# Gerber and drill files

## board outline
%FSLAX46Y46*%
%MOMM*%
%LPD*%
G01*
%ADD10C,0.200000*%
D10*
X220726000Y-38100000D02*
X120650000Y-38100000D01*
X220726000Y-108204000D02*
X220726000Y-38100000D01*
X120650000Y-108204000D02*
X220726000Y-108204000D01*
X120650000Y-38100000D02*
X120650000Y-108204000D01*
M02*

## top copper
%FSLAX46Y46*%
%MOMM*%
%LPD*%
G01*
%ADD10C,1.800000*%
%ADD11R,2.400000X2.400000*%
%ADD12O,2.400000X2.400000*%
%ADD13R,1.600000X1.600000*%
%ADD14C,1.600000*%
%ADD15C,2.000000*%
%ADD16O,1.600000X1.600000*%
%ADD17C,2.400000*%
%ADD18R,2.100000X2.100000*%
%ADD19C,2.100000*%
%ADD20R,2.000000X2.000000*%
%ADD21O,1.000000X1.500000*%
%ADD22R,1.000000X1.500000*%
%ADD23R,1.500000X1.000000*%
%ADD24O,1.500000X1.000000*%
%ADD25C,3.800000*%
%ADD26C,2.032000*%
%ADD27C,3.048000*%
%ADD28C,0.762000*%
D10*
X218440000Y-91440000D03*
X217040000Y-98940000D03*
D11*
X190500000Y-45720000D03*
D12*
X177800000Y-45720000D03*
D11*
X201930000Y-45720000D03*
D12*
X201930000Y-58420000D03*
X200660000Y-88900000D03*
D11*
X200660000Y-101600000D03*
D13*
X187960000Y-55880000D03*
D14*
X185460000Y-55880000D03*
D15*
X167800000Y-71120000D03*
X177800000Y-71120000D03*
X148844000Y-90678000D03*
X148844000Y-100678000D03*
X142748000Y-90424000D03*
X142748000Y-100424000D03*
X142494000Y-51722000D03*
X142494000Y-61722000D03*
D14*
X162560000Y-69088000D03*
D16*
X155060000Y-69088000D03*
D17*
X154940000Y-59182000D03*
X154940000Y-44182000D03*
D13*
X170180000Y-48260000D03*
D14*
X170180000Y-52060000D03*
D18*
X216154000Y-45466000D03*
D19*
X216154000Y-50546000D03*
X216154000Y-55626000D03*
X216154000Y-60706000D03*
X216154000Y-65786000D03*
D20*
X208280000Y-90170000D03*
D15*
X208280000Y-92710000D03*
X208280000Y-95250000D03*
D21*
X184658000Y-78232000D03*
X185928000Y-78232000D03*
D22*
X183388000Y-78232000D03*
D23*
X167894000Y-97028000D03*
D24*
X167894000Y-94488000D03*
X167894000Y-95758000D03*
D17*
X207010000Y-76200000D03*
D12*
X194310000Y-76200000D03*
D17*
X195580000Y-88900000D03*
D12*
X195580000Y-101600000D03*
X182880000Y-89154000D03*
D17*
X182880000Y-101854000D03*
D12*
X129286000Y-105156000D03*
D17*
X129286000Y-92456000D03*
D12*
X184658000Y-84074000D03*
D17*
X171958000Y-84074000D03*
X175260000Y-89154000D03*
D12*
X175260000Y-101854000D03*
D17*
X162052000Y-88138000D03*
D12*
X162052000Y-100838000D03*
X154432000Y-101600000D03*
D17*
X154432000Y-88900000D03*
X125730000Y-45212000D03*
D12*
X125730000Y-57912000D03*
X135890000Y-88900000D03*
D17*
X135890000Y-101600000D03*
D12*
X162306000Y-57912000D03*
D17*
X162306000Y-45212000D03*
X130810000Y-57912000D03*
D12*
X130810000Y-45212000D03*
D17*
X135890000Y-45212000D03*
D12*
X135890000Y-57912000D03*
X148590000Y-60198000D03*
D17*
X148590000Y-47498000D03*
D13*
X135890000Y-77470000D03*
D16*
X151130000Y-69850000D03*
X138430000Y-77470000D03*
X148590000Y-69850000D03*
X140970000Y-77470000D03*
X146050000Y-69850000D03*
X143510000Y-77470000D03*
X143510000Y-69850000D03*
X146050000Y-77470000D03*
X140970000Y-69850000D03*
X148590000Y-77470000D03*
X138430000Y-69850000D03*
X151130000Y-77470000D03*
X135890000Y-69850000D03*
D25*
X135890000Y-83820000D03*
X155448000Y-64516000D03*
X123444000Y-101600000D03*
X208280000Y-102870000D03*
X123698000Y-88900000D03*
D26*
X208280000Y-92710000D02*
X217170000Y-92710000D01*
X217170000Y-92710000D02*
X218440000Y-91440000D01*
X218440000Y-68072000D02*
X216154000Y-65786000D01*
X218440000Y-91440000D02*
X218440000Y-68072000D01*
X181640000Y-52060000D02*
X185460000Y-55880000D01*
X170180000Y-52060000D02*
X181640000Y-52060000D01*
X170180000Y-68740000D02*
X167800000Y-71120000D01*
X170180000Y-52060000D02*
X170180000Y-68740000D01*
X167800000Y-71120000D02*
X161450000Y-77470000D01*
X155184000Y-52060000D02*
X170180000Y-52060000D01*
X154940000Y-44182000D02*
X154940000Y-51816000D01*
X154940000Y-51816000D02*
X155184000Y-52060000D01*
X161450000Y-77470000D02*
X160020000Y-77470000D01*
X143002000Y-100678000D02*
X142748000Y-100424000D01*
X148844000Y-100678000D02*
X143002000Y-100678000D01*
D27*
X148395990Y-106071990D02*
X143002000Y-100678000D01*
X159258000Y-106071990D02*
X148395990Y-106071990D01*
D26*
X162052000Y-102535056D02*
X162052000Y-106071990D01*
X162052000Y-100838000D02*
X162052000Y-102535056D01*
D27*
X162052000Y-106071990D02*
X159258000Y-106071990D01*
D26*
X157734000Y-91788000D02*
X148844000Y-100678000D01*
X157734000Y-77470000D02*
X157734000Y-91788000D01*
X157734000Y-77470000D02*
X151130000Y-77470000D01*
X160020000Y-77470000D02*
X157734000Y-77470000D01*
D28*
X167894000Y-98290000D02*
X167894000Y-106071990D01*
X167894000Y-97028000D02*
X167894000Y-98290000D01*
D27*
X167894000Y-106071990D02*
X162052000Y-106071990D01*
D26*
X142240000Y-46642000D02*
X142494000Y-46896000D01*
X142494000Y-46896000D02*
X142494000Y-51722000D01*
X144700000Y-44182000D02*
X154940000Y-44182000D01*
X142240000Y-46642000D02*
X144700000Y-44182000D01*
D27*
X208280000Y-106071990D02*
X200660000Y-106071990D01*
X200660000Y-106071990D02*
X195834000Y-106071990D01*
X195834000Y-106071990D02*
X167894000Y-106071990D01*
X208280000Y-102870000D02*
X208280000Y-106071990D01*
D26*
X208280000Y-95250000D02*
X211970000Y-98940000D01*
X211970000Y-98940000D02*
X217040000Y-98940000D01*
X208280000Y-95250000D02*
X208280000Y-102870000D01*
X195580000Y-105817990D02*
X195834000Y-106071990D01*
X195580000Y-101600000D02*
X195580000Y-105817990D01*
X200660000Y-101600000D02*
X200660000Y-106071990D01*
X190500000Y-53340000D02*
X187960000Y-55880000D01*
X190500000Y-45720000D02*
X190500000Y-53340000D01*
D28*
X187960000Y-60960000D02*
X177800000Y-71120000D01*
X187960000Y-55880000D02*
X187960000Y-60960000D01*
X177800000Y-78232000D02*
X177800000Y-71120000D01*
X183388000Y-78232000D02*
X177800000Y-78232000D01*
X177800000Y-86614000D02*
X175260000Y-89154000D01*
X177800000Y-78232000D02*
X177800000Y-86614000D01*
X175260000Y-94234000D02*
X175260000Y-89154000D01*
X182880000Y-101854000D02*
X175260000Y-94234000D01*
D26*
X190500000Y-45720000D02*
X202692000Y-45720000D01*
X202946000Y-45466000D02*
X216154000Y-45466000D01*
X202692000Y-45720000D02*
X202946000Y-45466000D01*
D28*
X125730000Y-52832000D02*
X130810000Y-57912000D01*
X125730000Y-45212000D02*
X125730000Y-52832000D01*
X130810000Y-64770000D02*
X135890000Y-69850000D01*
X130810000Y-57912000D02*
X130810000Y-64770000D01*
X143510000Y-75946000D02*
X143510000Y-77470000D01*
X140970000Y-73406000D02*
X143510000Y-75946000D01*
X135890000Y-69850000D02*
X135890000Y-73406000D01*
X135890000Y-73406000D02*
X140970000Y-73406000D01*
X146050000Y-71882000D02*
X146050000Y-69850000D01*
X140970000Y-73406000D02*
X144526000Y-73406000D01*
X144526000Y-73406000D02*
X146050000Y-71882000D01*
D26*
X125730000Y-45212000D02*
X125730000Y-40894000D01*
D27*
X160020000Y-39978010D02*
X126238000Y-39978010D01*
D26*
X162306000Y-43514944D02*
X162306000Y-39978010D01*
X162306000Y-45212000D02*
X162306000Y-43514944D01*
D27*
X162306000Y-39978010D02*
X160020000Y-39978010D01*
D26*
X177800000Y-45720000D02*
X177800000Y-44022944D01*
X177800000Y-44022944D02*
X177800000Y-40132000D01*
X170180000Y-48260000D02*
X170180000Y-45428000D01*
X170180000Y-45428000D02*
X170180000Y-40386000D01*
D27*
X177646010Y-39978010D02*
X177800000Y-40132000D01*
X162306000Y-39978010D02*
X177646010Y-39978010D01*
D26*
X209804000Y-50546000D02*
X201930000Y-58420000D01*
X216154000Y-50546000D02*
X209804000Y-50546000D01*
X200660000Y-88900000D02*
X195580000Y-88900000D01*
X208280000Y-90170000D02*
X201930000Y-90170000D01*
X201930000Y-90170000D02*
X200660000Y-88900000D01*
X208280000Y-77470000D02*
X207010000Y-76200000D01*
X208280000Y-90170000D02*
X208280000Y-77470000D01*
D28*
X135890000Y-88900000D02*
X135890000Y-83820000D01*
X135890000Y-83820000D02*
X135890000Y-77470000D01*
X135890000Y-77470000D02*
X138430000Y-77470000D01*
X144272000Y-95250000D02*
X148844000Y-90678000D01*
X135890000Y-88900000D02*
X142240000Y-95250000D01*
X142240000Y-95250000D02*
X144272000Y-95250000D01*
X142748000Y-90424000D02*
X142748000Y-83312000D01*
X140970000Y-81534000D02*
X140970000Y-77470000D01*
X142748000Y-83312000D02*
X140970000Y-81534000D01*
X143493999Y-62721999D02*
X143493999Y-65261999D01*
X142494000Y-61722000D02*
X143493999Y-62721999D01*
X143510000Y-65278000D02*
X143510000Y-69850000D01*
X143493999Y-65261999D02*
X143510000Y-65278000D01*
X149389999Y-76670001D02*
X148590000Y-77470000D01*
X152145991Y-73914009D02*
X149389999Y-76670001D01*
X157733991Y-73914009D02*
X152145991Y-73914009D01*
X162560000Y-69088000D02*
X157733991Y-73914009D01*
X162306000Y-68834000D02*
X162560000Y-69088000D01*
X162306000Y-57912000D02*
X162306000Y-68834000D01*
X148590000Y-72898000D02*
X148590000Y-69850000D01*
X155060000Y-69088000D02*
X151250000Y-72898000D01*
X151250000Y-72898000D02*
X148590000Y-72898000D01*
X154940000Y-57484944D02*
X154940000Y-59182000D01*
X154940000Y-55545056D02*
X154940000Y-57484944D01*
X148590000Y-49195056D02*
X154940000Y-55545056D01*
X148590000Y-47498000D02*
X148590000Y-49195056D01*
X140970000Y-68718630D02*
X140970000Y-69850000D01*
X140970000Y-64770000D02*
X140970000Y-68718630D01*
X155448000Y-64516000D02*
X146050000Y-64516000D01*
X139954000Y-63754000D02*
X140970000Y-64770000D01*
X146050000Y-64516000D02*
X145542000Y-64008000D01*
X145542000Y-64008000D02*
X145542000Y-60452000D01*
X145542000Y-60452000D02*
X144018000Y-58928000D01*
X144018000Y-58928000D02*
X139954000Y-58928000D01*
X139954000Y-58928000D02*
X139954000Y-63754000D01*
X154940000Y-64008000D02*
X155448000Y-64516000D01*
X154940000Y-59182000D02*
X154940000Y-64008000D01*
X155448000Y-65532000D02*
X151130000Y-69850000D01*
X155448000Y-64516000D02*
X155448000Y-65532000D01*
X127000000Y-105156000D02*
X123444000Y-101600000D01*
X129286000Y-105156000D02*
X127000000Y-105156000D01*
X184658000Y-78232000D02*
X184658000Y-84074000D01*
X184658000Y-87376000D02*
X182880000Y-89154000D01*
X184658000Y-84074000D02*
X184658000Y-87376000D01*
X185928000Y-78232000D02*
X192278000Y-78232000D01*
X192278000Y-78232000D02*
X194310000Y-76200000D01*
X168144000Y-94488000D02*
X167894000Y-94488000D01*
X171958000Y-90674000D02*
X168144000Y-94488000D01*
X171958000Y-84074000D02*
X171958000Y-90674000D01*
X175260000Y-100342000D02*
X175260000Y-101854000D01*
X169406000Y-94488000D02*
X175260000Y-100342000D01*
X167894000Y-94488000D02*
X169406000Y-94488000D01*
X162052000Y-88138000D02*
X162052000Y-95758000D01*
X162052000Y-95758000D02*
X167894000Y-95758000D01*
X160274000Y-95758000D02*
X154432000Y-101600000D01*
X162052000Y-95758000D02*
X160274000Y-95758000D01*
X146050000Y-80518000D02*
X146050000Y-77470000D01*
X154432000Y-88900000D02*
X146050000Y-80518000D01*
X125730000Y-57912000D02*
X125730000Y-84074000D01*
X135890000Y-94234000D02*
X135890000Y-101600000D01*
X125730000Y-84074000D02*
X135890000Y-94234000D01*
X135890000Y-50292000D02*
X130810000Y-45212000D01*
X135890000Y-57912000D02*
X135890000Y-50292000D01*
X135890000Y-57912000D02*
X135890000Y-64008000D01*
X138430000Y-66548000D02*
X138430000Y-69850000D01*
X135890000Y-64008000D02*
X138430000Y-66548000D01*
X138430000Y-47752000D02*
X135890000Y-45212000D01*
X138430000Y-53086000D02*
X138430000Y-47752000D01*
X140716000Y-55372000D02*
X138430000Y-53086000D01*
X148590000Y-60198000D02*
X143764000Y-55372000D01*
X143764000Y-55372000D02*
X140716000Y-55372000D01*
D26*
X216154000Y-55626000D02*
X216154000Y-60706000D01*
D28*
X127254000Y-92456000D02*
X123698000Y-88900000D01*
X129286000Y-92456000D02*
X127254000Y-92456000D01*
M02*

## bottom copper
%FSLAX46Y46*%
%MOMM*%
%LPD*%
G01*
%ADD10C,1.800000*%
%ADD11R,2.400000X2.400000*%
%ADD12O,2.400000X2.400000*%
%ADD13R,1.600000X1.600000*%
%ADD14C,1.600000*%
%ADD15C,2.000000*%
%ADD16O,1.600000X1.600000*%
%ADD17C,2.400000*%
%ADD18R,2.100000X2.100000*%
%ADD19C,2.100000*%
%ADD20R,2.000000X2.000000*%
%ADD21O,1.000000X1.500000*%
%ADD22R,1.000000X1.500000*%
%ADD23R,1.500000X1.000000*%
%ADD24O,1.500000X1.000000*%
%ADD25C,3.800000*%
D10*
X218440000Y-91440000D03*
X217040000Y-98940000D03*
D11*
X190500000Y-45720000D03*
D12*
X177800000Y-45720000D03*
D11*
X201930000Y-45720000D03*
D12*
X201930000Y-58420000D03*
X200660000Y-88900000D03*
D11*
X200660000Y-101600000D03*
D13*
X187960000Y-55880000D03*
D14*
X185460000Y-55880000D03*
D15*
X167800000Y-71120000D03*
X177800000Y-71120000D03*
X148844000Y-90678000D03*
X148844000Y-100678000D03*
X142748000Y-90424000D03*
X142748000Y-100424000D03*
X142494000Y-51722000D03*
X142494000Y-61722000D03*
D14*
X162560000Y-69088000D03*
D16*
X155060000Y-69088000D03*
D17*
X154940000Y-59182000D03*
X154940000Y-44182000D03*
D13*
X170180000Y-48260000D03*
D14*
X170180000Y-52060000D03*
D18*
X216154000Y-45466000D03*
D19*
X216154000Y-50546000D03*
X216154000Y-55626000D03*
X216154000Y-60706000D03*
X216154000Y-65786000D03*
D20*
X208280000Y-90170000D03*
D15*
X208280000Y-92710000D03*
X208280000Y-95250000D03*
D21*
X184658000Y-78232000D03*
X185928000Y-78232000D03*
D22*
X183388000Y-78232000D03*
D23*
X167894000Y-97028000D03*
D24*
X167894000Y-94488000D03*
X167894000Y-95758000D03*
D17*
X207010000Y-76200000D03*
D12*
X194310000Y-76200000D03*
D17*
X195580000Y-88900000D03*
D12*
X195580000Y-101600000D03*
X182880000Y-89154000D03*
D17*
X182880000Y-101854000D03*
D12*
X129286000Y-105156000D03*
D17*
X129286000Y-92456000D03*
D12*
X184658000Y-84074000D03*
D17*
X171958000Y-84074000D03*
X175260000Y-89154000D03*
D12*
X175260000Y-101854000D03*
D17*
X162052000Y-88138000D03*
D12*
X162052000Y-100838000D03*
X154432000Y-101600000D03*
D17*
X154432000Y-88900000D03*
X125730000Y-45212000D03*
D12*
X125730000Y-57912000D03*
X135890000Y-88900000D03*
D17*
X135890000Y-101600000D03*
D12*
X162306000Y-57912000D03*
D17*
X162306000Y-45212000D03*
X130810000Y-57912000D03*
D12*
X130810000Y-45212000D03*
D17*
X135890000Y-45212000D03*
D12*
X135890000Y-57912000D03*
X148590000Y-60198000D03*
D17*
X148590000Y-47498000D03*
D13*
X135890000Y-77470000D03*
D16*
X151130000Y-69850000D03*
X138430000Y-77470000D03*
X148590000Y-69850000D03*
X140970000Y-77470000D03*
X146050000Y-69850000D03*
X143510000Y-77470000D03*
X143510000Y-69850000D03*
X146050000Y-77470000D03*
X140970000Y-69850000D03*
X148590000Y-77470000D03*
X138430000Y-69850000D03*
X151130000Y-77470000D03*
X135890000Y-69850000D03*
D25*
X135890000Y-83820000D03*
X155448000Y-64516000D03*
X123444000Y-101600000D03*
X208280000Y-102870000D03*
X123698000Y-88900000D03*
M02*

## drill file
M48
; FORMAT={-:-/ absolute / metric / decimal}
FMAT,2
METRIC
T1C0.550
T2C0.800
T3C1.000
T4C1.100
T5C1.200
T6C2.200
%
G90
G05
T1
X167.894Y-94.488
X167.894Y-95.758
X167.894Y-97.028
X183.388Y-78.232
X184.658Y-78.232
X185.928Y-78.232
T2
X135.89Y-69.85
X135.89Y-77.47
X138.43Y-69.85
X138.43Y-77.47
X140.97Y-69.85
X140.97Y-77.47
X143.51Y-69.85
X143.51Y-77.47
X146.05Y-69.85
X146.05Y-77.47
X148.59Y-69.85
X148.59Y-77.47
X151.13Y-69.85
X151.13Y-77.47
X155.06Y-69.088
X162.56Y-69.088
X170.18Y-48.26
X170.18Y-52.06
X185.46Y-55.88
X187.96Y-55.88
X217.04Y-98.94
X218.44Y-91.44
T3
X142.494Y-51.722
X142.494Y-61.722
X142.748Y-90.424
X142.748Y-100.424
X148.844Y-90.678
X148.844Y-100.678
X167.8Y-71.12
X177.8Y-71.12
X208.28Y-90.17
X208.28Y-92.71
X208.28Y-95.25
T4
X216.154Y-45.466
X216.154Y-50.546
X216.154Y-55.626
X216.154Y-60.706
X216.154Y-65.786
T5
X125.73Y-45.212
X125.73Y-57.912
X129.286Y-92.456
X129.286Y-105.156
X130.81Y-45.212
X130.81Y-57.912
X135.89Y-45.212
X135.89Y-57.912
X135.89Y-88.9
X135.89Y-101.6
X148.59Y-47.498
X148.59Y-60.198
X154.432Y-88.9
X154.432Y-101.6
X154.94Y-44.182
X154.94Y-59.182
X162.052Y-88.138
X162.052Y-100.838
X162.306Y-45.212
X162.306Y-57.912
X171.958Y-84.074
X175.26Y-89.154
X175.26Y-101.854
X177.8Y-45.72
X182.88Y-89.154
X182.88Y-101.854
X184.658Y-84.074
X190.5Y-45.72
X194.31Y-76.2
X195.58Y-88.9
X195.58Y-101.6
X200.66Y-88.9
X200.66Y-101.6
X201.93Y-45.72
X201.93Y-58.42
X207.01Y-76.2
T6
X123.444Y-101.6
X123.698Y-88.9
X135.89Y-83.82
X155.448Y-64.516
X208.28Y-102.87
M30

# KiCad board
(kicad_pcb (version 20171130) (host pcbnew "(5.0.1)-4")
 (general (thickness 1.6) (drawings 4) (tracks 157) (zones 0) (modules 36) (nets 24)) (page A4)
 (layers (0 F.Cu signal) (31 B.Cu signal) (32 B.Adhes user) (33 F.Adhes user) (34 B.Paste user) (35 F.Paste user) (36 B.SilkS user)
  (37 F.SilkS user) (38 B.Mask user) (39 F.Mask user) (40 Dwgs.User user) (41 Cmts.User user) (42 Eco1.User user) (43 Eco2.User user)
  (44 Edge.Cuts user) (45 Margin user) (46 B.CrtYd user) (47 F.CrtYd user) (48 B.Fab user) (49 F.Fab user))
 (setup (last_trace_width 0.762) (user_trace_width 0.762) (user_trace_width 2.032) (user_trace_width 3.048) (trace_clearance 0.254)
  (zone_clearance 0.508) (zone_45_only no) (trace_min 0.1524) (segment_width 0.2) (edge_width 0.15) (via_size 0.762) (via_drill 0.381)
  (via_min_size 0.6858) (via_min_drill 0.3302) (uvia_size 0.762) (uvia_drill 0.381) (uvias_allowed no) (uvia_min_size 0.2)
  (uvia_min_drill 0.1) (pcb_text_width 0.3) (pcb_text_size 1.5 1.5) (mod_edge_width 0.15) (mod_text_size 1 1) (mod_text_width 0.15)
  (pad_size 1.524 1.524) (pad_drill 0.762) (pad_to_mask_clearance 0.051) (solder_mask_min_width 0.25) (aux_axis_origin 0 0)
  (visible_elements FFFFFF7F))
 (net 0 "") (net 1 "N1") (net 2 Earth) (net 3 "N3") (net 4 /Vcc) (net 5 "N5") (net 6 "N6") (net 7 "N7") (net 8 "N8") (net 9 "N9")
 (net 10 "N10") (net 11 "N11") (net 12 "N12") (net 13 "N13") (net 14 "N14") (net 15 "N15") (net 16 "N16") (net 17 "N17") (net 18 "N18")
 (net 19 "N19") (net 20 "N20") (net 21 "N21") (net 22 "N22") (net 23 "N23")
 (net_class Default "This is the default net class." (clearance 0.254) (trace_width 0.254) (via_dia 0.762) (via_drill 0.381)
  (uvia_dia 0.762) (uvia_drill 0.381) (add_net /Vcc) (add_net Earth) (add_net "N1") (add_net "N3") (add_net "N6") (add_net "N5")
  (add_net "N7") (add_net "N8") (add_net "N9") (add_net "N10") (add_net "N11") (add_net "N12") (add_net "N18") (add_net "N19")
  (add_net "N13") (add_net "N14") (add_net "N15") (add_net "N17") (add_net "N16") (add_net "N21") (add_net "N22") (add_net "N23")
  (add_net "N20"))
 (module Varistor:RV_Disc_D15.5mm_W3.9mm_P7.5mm (layer F.Cu) (at 218.44 91.44 270)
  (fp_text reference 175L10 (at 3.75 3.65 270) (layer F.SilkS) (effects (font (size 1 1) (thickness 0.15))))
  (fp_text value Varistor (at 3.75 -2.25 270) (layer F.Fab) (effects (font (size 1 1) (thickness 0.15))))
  (pad 1 thru_hole circle (at 0 0 270) (size 1.8 1.8) (drill 0.8) (layers *.Cu *.Mask) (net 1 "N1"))
  (pad 2 thru_hole circle (at 7.5 1.4 270) (size 1.8 1.8) (drill 0.8) (layers *.Cu *.Mask) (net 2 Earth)))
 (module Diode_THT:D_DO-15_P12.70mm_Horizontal (layer F.Cu) (at 190.5 45.72 180)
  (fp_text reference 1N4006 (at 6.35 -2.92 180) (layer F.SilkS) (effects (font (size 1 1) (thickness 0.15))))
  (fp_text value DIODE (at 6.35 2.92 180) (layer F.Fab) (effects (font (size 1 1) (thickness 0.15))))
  (pad 1 thru_hole rect (at 0 0 180) (size 2.4 2.4) (drill 1.2) (layers *.Cu *.Mask) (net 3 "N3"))
  (pad 2 thru_hole oval (at 12.7 0 180) (size 2.4 2.4) (drill 1.2) (layers *.Cu *.Mask) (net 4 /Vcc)))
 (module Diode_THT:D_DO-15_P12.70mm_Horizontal (layer F.Cu) (at 201.93 45.72 270)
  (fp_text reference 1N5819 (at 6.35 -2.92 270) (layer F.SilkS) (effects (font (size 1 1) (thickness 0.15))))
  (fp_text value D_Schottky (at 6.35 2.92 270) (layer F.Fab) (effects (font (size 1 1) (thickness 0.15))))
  (pad 1 thru_hole rect (at 0 0 270) (size 2.4 2.4) (drill 1.2) (layers *.Cu *.Mask) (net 3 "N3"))
  (pad 2 thru_hole oval (at 12.7 0 270) (size 2.4 2.4) (drill 1.2) (layers *.Cu *.Mask) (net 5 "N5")))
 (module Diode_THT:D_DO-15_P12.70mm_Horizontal (layer F.Cu) (at 200.66 101.6 90)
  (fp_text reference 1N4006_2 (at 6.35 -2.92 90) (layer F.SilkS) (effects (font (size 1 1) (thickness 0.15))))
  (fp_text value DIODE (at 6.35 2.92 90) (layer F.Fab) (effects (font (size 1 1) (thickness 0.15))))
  (pad 2 thru_hole oval (at 12.7 0 90) (size 2.4 2.4) (drill 1.2) (layers *.Cu *.Mask) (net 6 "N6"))
  (pad 1 thru_hole rect (at 0 0 90) (size 2.4 2.4) (drill 1.2) (layers *.Cu *.Mask) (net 2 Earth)))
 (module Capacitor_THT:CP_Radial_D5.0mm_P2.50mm (layer F.Cu) (at 187.96 55.88 180)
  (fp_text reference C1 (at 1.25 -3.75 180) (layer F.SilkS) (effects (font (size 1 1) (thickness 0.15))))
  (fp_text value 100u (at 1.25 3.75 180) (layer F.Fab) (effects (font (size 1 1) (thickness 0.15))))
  (pad 1 thru_hole rect (at 0 0 180) (size 1.6 1.6) (drill 0.8) (layers *.Cu *.Mask) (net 3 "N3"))
  (pad 2 thru_hole circle (at 2.5 0 180) (size 1.6 1.6) (drill 0.8) (layers *.Cu *.Mask) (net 2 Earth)))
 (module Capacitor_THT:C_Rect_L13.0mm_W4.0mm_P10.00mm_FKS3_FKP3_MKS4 (layer F.Cu) (at 177.8 71.12 180)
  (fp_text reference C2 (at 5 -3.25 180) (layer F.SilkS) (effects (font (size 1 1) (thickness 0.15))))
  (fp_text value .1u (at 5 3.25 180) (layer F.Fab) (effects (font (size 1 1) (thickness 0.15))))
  (pad 2 thru_hole circle (at 10 0 180) (size 2 2) (drill 1) (layers *.Cu *.Mask) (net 2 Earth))
  (pad 1 thru_hole circle (at 0 0 180) (size 2 2) (drill 1) (layers *.Cu *.Mask) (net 3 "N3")))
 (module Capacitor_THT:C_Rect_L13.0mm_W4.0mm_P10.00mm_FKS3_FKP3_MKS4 (layer F.Cu) (at 148.844 90.678 270)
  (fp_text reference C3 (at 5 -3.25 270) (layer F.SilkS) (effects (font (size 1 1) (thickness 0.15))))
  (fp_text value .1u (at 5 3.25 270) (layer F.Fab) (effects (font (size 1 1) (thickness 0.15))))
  (pad 1 thru_hole circle (at 0 0 270) (size 2 2) (drill 1) (layers *.Cu *.Mask) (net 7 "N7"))
  (pad 2 thru_hole circle (at 10 0 270) (size 2 2) (drill 1) (layers *.Cu *.Mask) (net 2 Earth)))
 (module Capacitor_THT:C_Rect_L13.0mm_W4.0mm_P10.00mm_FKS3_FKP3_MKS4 (layer F.Cu) (at 142.748 90.424 270)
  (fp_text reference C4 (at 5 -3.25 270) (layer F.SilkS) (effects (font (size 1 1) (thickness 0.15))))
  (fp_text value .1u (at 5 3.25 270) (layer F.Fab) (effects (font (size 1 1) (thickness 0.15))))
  (pad 1 thru_hole circle (at 0 0 270) (size 2 2) (drill 1) (layers *.Cu *.Mask) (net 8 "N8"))
  (pad 2 thru_hole circle (at 10 0 270) (size 2 2) (drill 1) (layers *.Cu *.Mask) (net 2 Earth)))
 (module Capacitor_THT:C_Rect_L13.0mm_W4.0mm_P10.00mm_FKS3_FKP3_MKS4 (layer F.Cu) (at 142.494 61.722 90)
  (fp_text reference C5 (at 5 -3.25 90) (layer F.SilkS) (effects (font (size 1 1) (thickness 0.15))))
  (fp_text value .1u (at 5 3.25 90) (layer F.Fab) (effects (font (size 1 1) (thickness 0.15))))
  (pad 2 thru_hole circle (at 10 0 90) (size 2 2) (drill 1) (layers *.Cu *.Mask) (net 2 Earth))
  (pad 1 thru_hole circle (at 0 0 90) (size 2 2) (drill 1) (layers *.Cu *.Mask) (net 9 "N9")))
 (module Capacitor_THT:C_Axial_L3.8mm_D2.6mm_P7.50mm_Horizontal (layer F.Cu) (at 162.56 69.088 180)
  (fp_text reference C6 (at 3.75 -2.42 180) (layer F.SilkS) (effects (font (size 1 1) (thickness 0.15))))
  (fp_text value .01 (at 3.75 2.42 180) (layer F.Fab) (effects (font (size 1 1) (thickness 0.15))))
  (pad 1 thru_hole circle (at 0 0 180) (size 1.6 1.6) (drill 0.8) (layers *.Cu *.Mask) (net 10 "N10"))
  (pad 2 thru_hole oval (at 7.5 0 180) (size 1.6 1.6) (drill 0.8) (layers *.Cu *.Mask) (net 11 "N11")))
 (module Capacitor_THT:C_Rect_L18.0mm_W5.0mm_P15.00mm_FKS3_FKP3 (layer F.Cu) (at 154.94 59.182 90)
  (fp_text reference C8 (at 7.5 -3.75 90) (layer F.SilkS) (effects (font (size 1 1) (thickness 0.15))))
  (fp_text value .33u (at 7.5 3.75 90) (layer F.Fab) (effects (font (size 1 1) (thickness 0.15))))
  (pad 1 thru_hole circle (at 0 0 90) (size 2.4 2.4) (drill 1.2) (layers *.Cu *.Mask) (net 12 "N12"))
  (pad 2 thru_hole circle (at 15 0 90) (size 2.4 2.4) (drill 1.2) (layers *.Cu *.Mask) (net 2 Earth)))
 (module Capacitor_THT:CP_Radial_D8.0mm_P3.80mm (layer F.Cu) (at 170.18 48.26 270)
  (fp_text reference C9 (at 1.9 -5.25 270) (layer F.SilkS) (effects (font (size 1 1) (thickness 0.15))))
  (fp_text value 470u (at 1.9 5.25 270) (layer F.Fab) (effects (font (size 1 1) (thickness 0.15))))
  (pad 1 thru_hole rect (at 0 0 270) (size 1.6 1.6) (drill 0.8) (layers *.Cu *.Mask) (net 4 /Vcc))
  (pad 2 thru_hole circle (at 3.8 0 270) (size 1.6 1.6) (drill 0.8) (layers *.Cu *.Mask) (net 2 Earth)))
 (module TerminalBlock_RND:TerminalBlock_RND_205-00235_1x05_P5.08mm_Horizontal (layer F.Cu) (at 216.154 45.466 270)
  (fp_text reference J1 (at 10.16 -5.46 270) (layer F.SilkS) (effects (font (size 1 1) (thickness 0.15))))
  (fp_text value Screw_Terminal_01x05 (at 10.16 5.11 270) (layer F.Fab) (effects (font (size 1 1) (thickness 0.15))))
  (pad 1 thru_hole rect (at 0 0 270) (size 2.1 2.1) (drill 1.1) (layers *.Cu *.Mask) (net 3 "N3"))
  (pad 2 thru_hole circle (at 5.08 0 270) (size 2.1 2.1) (drill 1.1) (layers *.Cu *.Mask) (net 5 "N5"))
  (pad 3 thru_hole circle (at 10.16 0 270) (size 2.1 2.1) (drill 1.1) (layers *.Cu *.Mask) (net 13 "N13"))
  (pad 4 thru_hole circle (at 15.24 0 270) (size 2.1 2.1) (drill 1.1) (layers *.Cu *.Mask) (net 13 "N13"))
  (pad 5 thru_hole circle (at 20.32 0 270) (size 2.1 2.1) (drill 1.1) (layers *.Cu *.Mask) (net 1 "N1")))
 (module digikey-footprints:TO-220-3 (layer F.Cu) (at 208.28 90.17 270)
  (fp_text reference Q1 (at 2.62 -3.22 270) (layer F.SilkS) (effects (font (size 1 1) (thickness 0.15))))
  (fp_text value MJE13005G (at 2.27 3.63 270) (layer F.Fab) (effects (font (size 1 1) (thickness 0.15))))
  (pad 1 thru_hole rect (at 0 0 270) (size 2 2) (drill 1) (layers *.Cu *.Mask) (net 6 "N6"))
  (pad 2 thru_hole circle (at 2.54 0 270) (size 2 2) (drill 1) (layers *.Cu *.Mask) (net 1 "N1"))
  (pad 3 thru_hole circle (at 5.08 0 270) (size 2 2) (drill 1) (layers *.Cu *.Mask) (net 2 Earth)))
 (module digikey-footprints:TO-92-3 (layer F.Cu) (at 183.388 78.232)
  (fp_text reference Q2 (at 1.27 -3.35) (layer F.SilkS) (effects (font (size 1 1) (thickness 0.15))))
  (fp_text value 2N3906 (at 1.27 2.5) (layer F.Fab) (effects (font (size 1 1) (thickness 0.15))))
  (pad 2 thru_hole oval (at 1.27 0 180) (size 1 1.5) (drill 0.55) (layers *.Cu *.Mask) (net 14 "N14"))
  (pad 3 thru_hole oval (at 2.54 0 180) (size 1 1.5) (drill 0.55) (layers *.Cu *.Mask) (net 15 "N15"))
  (pad 1 thru_hole rect (at 0 0 180) (size 1 1.5) (drill 0.55) (layers *.Cu *.Mask) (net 3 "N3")))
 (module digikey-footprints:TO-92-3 (layer F.Cu) (at 167.894 97.028 90)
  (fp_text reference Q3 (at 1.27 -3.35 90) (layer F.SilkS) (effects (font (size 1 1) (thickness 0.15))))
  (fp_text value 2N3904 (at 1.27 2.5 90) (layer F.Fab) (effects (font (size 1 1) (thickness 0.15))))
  (pad 1 thru_hole rect (at 0 0 270) (size 1 1.5) (drill 0.55) (layers *.Cu *.Mask) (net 2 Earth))
  (pad 3 thru_hole oval (at 2.54 0 270) (size 1 1.5) (drill 0.55) (layers *.Cu *.Mask) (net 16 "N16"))
  (pad 2 thru_hole oval (at 1.27 0 270) (size 1 1.5) (drill 0.55) (layers *.Cu *.Mask) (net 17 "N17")))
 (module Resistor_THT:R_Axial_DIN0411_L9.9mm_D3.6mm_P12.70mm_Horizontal (layer F.Cu) (at 207.01 76.2 180)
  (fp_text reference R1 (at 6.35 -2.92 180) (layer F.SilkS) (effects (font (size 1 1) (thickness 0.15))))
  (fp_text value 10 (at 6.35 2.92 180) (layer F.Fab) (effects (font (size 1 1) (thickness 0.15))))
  (pad 1 thru_hole circle (at 0 0 180) (size 2.4 2.4) (drill 1.2) (layers *.Cu *.Mask) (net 6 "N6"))
  (pad 2 thru_hole oval (at 12.7 0 180) (size 2.4 2.4) (drill 1.2) (layers *.Cu *.Mask) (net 15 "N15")))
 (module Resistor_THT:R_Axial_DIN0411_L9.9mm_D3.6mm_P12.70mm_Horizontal (layer F.Cu) (at 195.58 88.9 270)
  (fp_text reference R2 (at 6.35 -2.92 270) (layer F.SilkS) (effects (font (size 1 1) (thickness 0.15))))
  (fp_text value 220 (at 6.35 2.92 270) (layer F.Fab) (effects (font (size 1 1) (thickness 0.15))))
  (pad 1 thru_hole circle (at 0 0 270) (size 2.4 2.4) (drill 1.2) (layers *.Cu *.Mask) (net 6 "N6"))
  (pad 2 thru_hole oval (at 12.7 0 270) (size 2.4 2.4) (drill 1.2) (layers *.Cu *.Mask) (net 2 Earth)))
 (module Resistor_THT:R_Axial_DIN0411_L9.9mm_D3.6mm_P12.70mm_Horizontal (layer F.Cu) (at 182.88 101.854 90)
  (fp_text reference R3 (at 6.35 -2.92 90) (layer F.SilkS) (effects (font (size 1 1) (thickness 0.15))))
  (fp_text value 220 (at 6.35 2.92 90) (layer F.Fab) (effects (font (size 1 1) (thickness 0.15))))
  (pad 2 thru_hole oval (at 12.7 0 90) (size 2.4 2.4) (drill 1.2) (layers *.Cu *.Mask) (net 14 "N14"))
  (pad 1 thru_hole circle (at 0 0 90) (size 2.4 2.4) (drill 1.2) (layers *.Cu *.Mask) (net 3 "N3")))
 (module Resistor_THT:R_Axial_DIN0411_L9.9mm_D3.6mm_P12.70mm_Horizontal (layer F.Cu) (at 129.286 92.456 270)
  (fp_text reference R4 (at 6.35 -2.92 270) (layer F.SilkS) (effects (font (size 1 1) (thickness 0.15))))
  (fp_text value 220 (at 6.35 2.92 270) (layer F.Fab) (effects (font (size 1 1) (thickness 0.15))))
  (pad 2 thru_hole oval (at 12.7 0 270) (size 2.4 2.4) (drill 1.2) (layers *.Cu *.Mask) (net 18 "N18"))
  (pad 1 thru_hole circle (at 0 0 270) (size 2.4 2.4) (drill 1.2) (layers *.Cu *.Mask) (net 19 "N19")))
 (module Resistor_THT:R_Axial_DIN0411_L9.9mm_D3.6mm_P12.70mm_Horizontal (layer F.Cu) (at 171.958 84.074)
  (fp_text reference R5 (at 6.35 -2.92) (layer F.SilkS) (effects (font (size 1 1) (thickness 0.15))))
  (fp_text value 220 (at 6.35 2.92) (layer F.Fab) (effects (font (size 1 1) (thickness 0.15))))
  (pad 2 thru_hole oval (at 12.7 0) (size 2.4 2.4) (drill 1.2) (layers *.Cu *.Mask) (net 14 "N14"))
  (pad 1 thru_hole circle (at 0 0) (size 2.4 2.4) (drill 1.2) (layers *.Cu *.Mask) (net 16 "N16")))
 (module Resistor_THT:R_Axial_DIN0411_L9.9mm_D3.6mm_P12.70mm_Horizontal (layer F.Cu) (at 175.26 89.154 270)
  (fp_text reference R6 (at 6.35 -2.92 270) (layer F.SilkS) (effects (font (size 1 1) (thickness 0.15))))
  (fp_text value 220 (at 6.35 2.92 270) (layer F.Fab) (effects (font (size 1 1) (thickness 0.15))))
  (pad 1 thru_hole circle (at 0 0 270) (size 2.4 2.4) (drill 1.2) (layers *.Cu *.Mask) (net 3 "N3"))
  (pad 2 thru_hole oval (at 12.7 0 270) (size 2.4 2.4) (drill 1.2) (layers *.Cu *.Mask) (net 16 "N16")))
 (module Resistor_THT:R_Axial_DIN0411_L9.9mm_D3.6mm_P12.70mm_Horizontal (layer F.Cu) (at 162.052 88.138 270)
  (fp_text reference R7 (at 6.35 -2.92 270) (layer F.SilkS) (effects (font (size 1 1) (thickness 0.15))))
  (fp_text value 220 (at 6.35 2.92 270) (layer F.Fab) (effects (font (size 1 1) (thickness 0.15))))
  (pad 1 thru_hole circle (at 0 0 270) (size 2.4 2.4) (drill 1.2) (layers *.Cu *.Mask) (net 17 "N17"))
  (pad 2 thru_hole oval (at 12.7 0 270) (size 2.4 2.4) (drill 1.2) (layers *.Cu *.Mask) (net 2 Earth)))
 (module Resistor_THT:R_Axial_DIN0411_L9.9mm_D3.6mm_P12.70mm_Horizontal (layer F.Cu) (at 154.432 88.9 270)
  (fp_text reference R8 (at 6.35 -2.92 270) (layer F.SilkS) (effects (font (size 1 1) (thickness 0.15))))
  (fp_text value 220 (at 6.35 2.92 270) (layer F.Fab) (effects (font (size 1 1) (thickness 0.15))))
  (pad 2 thru_hole oval (at 12.7 0 270) (size 2.4 2.4) (drill 1.2) (layers *.Cu *.Mask) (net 17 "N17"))
  (pad 1 thru_hole circle (at 0 0 270) (size 2.4 2.4) (drill 1.2) (layers *.Cu *.Mask) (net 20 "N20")))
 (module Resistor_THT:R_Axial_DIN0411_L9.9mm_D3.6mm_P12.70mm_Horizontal (layer F.Cu) (at 125.73 45.212 270)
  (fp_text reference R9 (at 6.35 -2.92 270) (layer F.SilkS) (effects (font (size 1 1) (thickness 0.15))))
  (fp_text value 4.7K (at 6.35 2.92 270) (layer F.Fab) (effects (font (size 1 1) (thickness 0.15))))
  (pad 1 thru_hole circle (at 0 0 270) (size 2.4 2.4) (drill 1.2) (layers *.Cu *.Mask) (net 4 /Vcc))
  (pad 2 thru_hole oval (at 12.7 0 270) (size 2.4 2.4) (drill 1.2) (layers *.Cu *.Mask) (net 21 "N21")))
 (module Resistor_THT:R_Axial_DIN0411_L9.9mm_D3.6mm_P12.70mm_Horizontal (layer F.Cu) (at 135.89 101.6 90)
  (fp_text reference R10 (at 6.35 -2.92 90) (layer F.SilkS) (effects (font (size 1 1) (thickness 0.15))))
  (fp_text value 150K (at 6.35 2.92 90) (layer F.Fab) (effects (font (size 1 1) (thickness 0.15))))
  (pad 2 thru_hole oval (at 12.7 0 90) (size 2.4 2.4) (drill 1.2) (layers *.Cu *.Mask) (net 7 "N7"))
  (pad 1 thru_hole circle (at 0 0 90) (size 2.4 2.4) (drill 1.2) (layers *.Cu *.Mask) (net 21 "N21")))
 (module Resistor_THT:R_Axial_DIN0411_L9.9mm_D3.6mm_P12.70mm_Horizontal (layer F.Cu) (at 162.306 45.212 270)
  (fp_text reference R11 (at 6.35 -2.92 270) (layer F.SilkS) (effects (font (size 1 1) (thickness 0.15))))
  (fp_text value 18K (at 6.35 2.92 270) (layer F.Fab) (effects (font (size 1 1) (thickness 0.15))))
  (pad 2 thru_hole oval (at 12.7 0 270) (size 2.4 2.4) (drill 1.2) (layers *.Cu *.Mask) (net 10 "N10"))
  (pad 1 thru_hole circle (at 0 0 270) (size 2.4 2.4) (drill 1.2) (layers *.Cu *.Mask) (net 4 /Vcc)))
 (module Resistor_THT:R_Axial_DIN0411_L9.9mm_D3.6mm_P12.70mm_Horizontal (layer F.Cu) (at 130.81 57.912 90)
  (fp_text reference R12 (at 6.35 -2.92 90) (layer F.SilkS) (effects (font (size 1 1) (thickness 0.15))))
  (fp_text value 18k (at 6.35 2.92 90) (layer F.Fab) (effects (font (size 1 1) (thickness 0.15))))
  (pad 1 thru_hole circle (at 0 0 90) (size 2.4 2.4) (drill 1.2) (layers *.Cu *.Mask) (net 4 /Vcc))
  (pad 2 thru_hole oval (at 12.7 0 90) (size 2.4 2.4) (drill 1.2) (layers *.Cu *.Mask) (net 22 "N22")))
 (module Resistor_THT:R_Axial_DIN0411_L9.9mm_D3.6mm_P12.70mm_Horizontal (layer F.Cu) (at 135.89 45.212 270)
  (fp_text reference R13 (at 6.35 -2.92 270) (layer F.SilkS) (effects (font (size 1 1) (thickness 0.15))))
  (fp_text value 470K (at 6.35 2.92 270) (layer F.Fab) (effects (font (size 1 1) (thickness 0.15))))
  (pad 1 thru_hole circle (at 0 0 270) (size 2.4 2.4) (drill 1.2) (layers *.Cu *.Mask) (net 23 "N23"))
  (pad 2 thru_hole oval (at 12.7 0 270) (size 2.4 2.4) (drill 1.2) (layers *.Cu *.Mask) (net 22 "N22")))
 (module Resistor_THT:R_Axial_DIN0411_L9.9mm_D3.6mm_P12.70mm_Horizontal (layer F.Cu) (at 148.59 47.498 270)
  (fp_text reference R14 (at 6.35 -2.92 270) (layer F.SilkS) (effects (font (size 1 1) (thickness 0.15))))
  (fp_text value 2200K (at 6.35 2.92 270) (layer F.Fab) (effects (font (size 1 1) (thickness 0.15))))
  (pad 2 thru_hole oval (at 12.7 0 270) (size 2.4 2.4) (drill 1.2) (layers *.Cu *.Mask) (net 23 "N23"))
  (pad 1 thru_hole circle (at 0 0 270) (size 2.4 2.4) (drill 1.2) (layers *.Cu *.Mask) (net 12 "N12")))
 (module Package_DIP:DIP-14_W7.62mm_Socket (layer F.Cu) (at 135.89 77.47 90)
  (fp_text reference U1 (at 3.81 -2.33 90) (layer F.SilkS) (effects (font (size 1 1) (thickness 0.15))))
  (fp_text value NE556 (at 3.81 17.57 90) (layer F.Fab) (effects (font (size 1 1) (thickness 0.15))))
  (pad 1 thru_hole rect (at 0 0 90) (size 1.6 1.6) (drill 0.8) (layers *.Cu *.Mask) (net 7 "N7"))
  (pad 8 thru_hole oval (at 7.62 15.24 90) (size 1.6 1.6) (drill 0.8) (layers *.Cu *.Mask) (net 12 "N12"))
  (pad 2 thru_hole oval (at 0 2.54 90) (size 1.6 1.6) (drill 0.8) (layers *.Cu *.Mask) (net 7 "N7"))
  (pad 9 thru_hole oval (at 7.62 12.7 90) (size 1.6 1.6) (drill 0.8) (layers *.Cu *.Mask) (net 11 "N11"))
  (pad 3 thru_hole oval (at 0 5.08 90) (size 1.6 1.6) (drill 0.8) (layers *.Cu *.Mask) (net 8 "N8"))
  (pad 10 thru_hole oval (at 7.62 10.16 90) (size 1.6 1.6) (drill 0.8) (layers *.Cu *.Mask) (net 4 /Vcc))
  (pad 4 thru_hole oval (at 0 7.62 90) (size 1.6 1.6) (drill 0.8) (layers *.Cu *.Mask) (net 4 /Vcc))
  (pad 11 thru_hole oval (at 7.62 7.62 90) (size 1.6 1.6) (drill 0.8) (layers *.Cu *.Mask) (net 9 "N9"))
  (pad 5 thru_hole oval (at 0 10.16 90) (size 1.6 1.6) (drill 0.8) (layers *.Cu *.Mask) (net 20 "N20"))
  (pad 12 thru_hole oval (at 7.62 5.08 90) (size 1.6 1.6) (drill 0.8) (layers *.Cu *.Mask) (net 12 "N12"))
  (pad 6 thru_hole oval (at 0 12.7 90) (size 1.6 1.6) (drill 0.8) (layers *.Cu *.Mask) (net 10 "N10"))
  (pad 13 thru_hole oval (at 7.62 2.54 90) (size 1.6 1.6) (drill 0.8) (layers *.Cu *.Mask) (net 22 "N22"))
  (pad 7 thru_hole oval (at 0 15.24 90) (size 1.6 1.6) (drill 0.8) (layers *.Cu *.Mask) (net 2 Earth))
  (pad 14 thru_hole oval (at 7.62 0 90) (size 1.6 1.6) (drill 0.8) (layers *.Cu *.Mask) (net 4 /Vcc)))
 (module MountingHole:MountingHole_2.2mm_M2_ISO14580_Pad (layer F.Cu) (at 135.89 83.82)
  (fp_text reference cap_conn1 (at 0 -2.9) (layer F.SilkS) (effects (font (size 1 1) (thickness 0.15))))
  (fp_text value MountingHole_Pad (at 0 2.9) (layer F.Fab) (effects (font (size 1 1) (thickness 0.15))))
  (pad 1 thru_hole circle (at 0 0) (size 3.8 3.8) (drill 2.2) (layers *.Cu *.Mask) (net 7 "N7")))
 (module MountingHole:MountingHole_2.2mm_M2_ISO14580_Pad (layer F.Cu) (at 155.448 64.516)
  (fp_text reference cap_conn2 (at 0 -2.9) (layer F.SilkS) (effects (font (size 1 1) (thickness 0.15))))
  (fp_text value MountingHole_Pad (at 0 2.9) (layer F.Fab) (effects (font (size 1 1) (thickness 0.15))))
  (pad 1 thru_hole circle (at 0 0) (size 3.8 3.8) (drill 2.2) (layers *.Cu *.Mask) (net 12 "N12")))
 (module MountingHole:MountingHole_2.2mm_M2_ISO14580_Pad (layer F.Cu) (at 123.444 101.6)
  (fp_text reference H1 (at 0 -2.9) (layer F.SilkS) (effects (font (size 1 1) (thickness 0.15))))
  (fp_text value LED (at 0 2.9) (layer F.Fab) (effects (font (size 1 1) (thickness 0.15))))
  (pad 1 thru_hole circle (at 0 0) (size 3.8 3.8) (drill 2.2) (layers *.Cu *.Mask) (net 18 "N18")))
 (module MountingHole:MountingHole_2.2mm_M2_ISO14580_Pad (layer F.Cu) (at 208.28 102.87)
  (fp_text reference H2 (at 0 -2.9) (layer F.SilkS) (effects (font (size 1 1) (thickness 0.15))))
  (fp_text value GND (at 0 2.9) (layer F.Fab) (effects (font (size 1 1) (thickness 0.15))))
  (pad 1 thru_hole circle (at 0 0) (size 3.8 3.8) (drill 2.2) (layers *.Cu *.Mask) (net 2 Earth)))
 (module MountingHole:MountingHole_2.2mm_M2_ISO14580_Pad (layer F.Cu) (at 123.698 88.9)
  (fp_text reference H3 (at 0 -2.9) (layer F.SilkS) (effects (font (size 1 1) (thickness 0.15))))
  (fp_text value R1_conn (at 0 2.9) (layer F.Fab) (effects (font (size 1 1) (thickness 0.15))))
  (pad 1 thru_hole circle (at 0 0) (size 3.8 3.8) (drill 2.2) (layers *.Cu *.Mask) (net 19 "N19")))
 (gr_line (start 220.726 38.1) (end 120.65 38.1) (layer Edge.Cuts) (width 0.2))
 (gr_line (start 220.726 108.204) (end 220.726 38.1) (layer Edge.Cuts) (width 0.2))
 (gr_line (start 120.65 108.204) (end 220.726 108.204) (layer Edge.Cuts) (width 0.2))
 (gr_line (start 120.65 38.1) (end 120.65 108.204) (layer Edge.Cuts) (width 0.2))
 (segment (start 208.28 92.71) (end 217.17 92.71) (width 2.032) (layer F.Cu) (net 1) (status 1000000))
 (segment (start 217.17 92.71) (end 218.44 91.44) (width 2.032) (layer F.Cu) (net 1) (status 1000000))
 (segment (start 218.44 68.072) (end 216.154 65.786) (width 2.032) (layer F.Cu) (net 1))
 (segment (start 218.44 91.44) (end 218.44 68.072) (width 2.032) (layer F.Cu) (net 1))
 (segment (start 181.64 52.06) (end 185.46 55.88) (width 2.032) (layer F.Cu) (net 2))
 (segment (start 170.18 52.06) (end 181.64 52.06) (width 2.032) (layer F.Cu) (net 2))
 (segment (start 170.18 68.74) (end 167.8 71.12) (width 2.032) (layer F.Cu) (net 2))
 (segment (start 170.18 52.06) (end 170.18 68.74) (width 2.032) (layer F.Cu) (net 2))
 (segment (start 167.8 71.12) (end 161.45 77.47) (width 2.032) (layer F.Cu) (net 2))
 (segment (start 155.184 52.06) (end 170.18 52.06) (width 2.032) (layer F.Cu) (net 2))
 (segment (start 154.94 44.182) (end 154.94 51.816) (width 2.032) (layer F.Cu) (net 2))
 (segment (start 154.94 51.816) (end 155.184 52.06) (width 2.032) (layer F.Cu) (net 2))
 (segment (start 161.45 77.47) (end 160.02 77.47) (width 2.032) (layer F.Cu) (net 2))
 (segment (start 143.002 100.678) (end 142.748 100.424) (width 2.032) (layer F.Cu) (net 2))
 (segment (start 148.844 100.678) (end 143.002 100.678) (width 2.032) (layer F.Cu) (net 2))
 (segment (start 148.39599 106.07199) (end 143.002 100.678) (width 3.048) (layer F.Cu) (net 2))
 (segment (start 159.258 106.07199) (end 148.39599 106.07199) (width 3.048) (layer F.Cu) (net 2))
 (segment (start 162.052 102.535056) (end 162.052 106.07199) (width 2.032) (layer F.Cu) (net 2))
 (segment (start 162.052 100.838) (end 162.052 102.535056) (width 2.032) (layer F.Cu) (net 2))
 (segment (start 162.052 106.07199) (end 159.258 106.07199) (width 3.048) (layer F.Cu) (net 2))
 (segment (start 157.734 91.788) (end 148.844 100.678) (width 2.032) (layer F.Cu) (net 2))
 (segment (start 157.734 77.47) (end 157.734 91.788) (width 2.032) (layer F.Cu) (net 2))
 (segment (start 157.734 77.47) (end 151.13 77.47) (width 2.032) (layer F.Cu) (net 2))
 (segment (start 160.02 77.47) (end 157.734 77.47) (width 2.032) (layer F.Cu) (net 2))
 (segment (start 167.894 98.29) (end 167.894 106.07199) (width 0.762) (layer F.Cu) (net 2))
 (segment (start 167.894 97.028) (end 167.894 98.29) (width 0.762) (layer F.Cu) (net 2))
 (segment (start 167.894 106.07199) (end 162.052 106.07199) (width 3.048) (layer F.Cu) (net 2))
 (segment (start 142.24 46.642) (end 142.494 46.896) (width 2.032) (layer F.Cu) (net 2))
 (segment (start 142.494 46.896) (end 142.494 51.722) (width 2.032) (layer F.Cu) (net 2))
 (segment (start 144.7 44.182) (end 154.94 44.182) (width 2.032) (layer F.Cu) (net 2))
 (segment (start 142.24 46.642) (end 144.7 44.182) (width 2.032) (layer F.Cu) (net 2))
 (segment (start 208.28 106.07199) (end 200.66 106.07199) (width 3.048) (layer F.Cu) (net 2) (status 1000000))
 (segment (start 200.66 106.07199) (end 195.834 106.07199) (width 3.048) (layer F.Cu) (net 2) (status 1000000))
 (segment (start 195.834 106.07199) (end 167.894 106.07199) (width 3.048) (layer F.Cu) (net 2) (status 1000000))
 (segment (start 208.28 102.87) (end 208.28 106.07199) (width 3.048) (layer F.Cu) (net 2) (status 1000000))
 (segment (start 208.28 95.25) (end 211.97 98.94) (width 2.032) (layer F.Cu) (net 2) (status 1000000))
 (segment (start 211.97 98.94) (end 217.04 98.94) (width 2.032) (layer F.Cu) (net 2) (status 1000000))
 (segment (start 208.28 95.25) (end 208.28 102.87) (width 2.032) (layer F.Cu) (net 2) (status 1000000))
 (segment (start 195.58 105.81799) (end 195.834 106.07199) (width 2.032) (layer F.Cu) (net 2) (status 1000000))
 (segment (start 195.58 101.6) (end 195.58 105.81799) (width 2.032) (layer F.Cu) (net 2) (status 1000000))
 (segment (start 200.66 101.6) (end 200.66 106.07199) (width 2.032) (layer F.Cu) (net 2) (status 1000000))
 (segment (start 190.5 53.34) (end 187.96 55.88) (width 2.032) (layer F.Cu) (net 3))
 (segment (start 190.5 45.72) (end 190.5 53.34) (width 2.032) (layer F.Cu) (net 3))
 (segment (start 187.96 60.96) (end 177.8 71.12) (width 0.762) (layer F.Cu) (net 3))
 (segment (start 187.96 55.88) (end 187.96 60.96) (width 0.762) (layer F.Cu) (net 3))
 (segment (start 177.8 78.232) (end 177.8 71.12) (width 0.762) (layer F.Cu) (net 3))
 (segment (start 183.388 78.232) (end 177.8 78.232) (width 0.762) (layer F.Cu) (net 3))
 (segment (start 177.8 86.614) (end 175.26 89.154) (width 0.762) (layer F.Cu) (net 3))
 (segment (start 177.8 78.232) (end 177.8 86.614) (width 0.762) (layer F.Cu) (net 3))
 (segment (start 175.26 94.234) (end 175.26 89.154) (width 0.762) (layer F.Cu) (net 3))
 (segment (start 182.88 101.854) (end 175.26 94.234) (width 0.762) (layer F.Cu) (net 3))
 (segment (start 190.5 45.72) (end 202.692 45.72) (width 2.032) (layer F.Cu) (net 3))
 (segment (start 202.946 45.466) (end 216.154 45.466) (width 2.032) (layer F.Cu) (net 3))
 (segment (start 202.692 45.72) (end 202.946 45.466) (width 2.032) (layer F.Cu) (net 3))
 (segment (start 125.73 52.832) (end 130.81 57.912) (width 0.762) (layer F.Cu) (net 4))
 (segment (start 125.73 45.212) (end 125.73 52.832) (width 0.762) (layer F.Cu) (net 4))
 (segment (start 130.81 64.77) (end 135.89 69.85) (width 0.762) (layer F.Cu) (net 4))
 (segment (start 130.81 57.912) (end 130.81 64.77) (width 0.762) (layer F.Cu) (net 4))
 (segment (start 143.51 75.946) (end 143.51 77.47) (width 0.762) (layer F.Cu) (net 4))
 (segment (start 140.97 73.406) (end 143.51 75.946) (width 0.762) (layer F.Cu) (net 4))
 (segment (start 135.89 69.85) (end 135.89 73.406) (width 0.762) (layer F.Cu) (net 4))
 (segment (start 135.89 73.406) (end 140.97 73.406) (width 0.762) (layer F.Cu) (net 4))
 (segment (start 146.05 71.882) (end 146.05 69.85) (width 0.762) (layer F.Cu) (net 4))
 (segment (start 140.97 73.406) (end 144.526 73.406) (width 0.762) (layer F.Cu) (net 4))
 (segment (start 144.526 73.406) (end 146.05 71.882) (width 0.762) (layer F.Cu) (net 4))
 (segment (start 125.73 45.212) (end 125.73 40.894) (width 2.032) (layer F.Cu) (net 4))
 (segment (start 160.02 39.97801) (end 126.238 39.97801) (width 3.048) (layer F.Cu) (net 4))
 (segment (start 162.306 43.514944) (end 162.306 39.97801) (width 2.032) (layer F.Cu) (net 4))
 (segment (start 162.306 45.212) (end 162.306 43.514944) (width 2.032) (layer F.Cu) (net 4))
 (segment (start 162.306 39.97801) (end 160.02 39.97801) (width 3.048) (layer F.Cu) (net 4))
 (segment (start 177.8 45.72) (end 177.8 44.022944) (width 2.032) (layer F.Cu) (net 4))
 (segment (start 177.8 44.022944) (end 177.8 40.132) (width 2.032) (layer F.Cu) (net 4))
 (segment (start 170.18 48.26) (end 170.18 45.428) (width 2.032) (layer F.Cu) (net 4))
 (segment (start 170.18 45.428) (end 170.18 40.386) (width 2.032) (layer F.Cu) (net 4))
 (segment (start 177.64601 39.97801) (end 177.8 40.132) (width 3.048) (layer F.Cu) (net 4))
 (segment (start 162.306 39.97801) (end 177.64601 39.97801) (width 3.048) (layer F.Cu) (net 4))
 (segment (start 209.804 50.546) (end 201.93 58.42) (width 2.032) (layer F.Cu) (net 5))
 (segment (start 216.154 50.546) (end 209.804 50.546) (width 2.032) (layer F.Cu) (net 5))
 (segment (start 200.66 88.9) (end 195.58 88.9) (width 2.032) (layer F.Cu) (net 6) (status 1000000))
 (segment (start 208.28 90.17) (end 201.93 90.17) (width 2.032) (layer F.Cu) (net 6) (status 1000000))
 (segment (start 201.93 90.17) (end 200.66 88.9) (width 2.032) (layer F.Cu) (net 6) (status 1000000))
 (segment (start 208.28 77.47) (end 207.01 76.2) (width 2.032) (layer F.Cu) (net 6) (status 1000000))
 (segment (start 208.28 90.17) (end 208.28 77.47) (width 2.032) (layer F.Cu) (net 6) (status 1000000))
 (segment (start 135.89 88.9) (end 135.89 83.82) (width 0.762) (layer F.Cu) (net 7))
 (segment (start 135.89 83.82) (end 135.89 77.47) (width 0.762) (layer F.Cu) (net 7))
 (segment (start 135.89 77.47) (end 138.43 77.47) (width 0.762) (layer F.Cu) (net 7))
 (segment (start 144.272 95.25) (end 148.844 90.678) (width 0.762) (layer F.Cu) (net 7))
 (segment (start 135.89 88.9) (end 142.24 95.25) (width 0.762) (layer F.Cu) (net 7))
 (segment (start 142.24 95.25) (end 144.272 95.25) (width 0.762) (layer F.Cu) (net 7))
 (segment (start 142.748 90.424) (end 142.748 83.312) (width 0.762) (layer F.Cu) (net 8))
 (segment (start 140.97 81.534) (end 140.97 77.47) (width 0.762) (layer F.Cu) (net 8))
 (segment (start 142.748 83.312) (end 140.97 81.534) (width 0.762) (layer F.Cu) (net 8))
 (segment (start 143.493999 62.721999) (end 143.493999 65.261999) (width 0.762) (layer F.Cu) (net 9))
 (segment (start 142.494 61.722) (end 143.493999 62.721999) (width 0.762) (layer F.Cu) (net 9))
 (segment (start 143.51 65.278) (end 143.51 69.85) (width 0.762) (layer F.Cu) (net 9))
 (segment (start 143.493999 65.261999) (end 143.51 65.278) (width 0.762) (layer F.Cu) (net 9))
 (segment (start 149.389999 76.670001) (end 148.59 77.47) (width 0.762) (layer F.Cu) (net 10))
 (segment (start 152.145991 73.914009) (end 149.389999 76.670001) (width 0.762) (layer F.Cu) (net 10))
 (segment (start 157.733991 73.914009) (end 152.145991 73.914009) (width 0.762) (layer F.Cu) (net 10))
 (segment (start 162.56 69.088) (end 157.733991 73.914009) (width 0.762) (layer F.Cu) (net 10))
 (segment (start 162.306 68.834) (end 162.56 69.088) (width 0.762) (layer F.Cu) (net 10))
 (segment (start 162.306 57.912) (end 162.306 68.834) (width 0.762) (layer F.Cu) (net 10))
 (segment (start 148.59 72.898) (end 148.59 69.85) (width 0.762) (layer F.Cu) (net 11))
 (segment (start 155.06 69.088) (end 151.25 72.898) (width 0.762) (layer F.Cu) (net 11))
 (segment (start 151.25 72.898) (end 148.59 72.898) (width 0.762) (layer F.Cu) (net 11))
 (segment (start 154.94 57.484944) (end 154.94 59.182) (width 0.762) (layer F.Cu) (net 12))
 (segment (start 154.94 55.545056) (end 154.94 57.484944) (width 0.762) (layer F.Cu) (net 12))
 (segment (start 148.59 49.195056) (end 154.94 55.545056) (width 0.762) (layer F.Cu) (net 12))
 (segment (start 148.59 47.498) (end 148.59 49.195056) (width 0.762) (layer F.Cu) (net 12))
 (segment (start 140.97 68.71863) (end 140.97 69.85) (width 0.762) (layer F.Cu) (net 12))
 (segment (start 140.97 64.77) (end 140.97 68.71863) (width 0.762) (layer F.Cu) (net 12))
 (segment (start 155.448 64.516) (end 146.05 64.516) (width 0.762) (layer F.Cu) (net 12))
 (segment (start 139.954 63.754) (end 140.97 64.77) (width 0.762) (layer F.Cu) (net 12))
 (segment (start 146.05 64.516) (end 145.542 64.008) (width 0.762) (layer F.Cu) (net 12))
 (segment (start 145.542 64.008) (end 145.542 60.452) (width 0.762) (layer F.Cu) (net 12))
 (segment (start 145.542 60.452) (end 144.018 58.928) (width 0.762) (layer F.Cu) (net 12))
 (segment (start 144.018 58.928) (end 139.954 58.928) (width 0.762) (layer F.Cu) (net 12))
 (segment (start 139.954 58.928) (end 139.954 63.754) (width 0.762) (layer F.Cu) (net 12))
 (segment (start 154.94 64.008) (end 155.448 64.516) (width 0.762) (layer F.Cu) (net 12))
 (segment (start 154.94 59.182) (end 154.94 64.008) (width 0.762) (layer F.Cu) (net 12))
 (segment (start 155.448 65.532) (end 151.13 69.85) (width 0.762) (layer F.Cu) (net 12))
 (segment (start 155.448 64.516) (end 155.448 65.532) (width 0.762) (layer F.Cu) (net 12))
 (segment (start 127 105.156) (end 123.444 101.6) (width 0.762) (layer F.Cu) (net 18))
 (segment (start 129.286 105.156) (end 127 105.156) (width 0.762) (layer F.Cu) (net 18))
 (segment (start 184.658 78.232) (end 184.658 84.074) (width 0.762) (layer F.Cu) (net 14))
 (segment (start 184.658 87.376) (end 182.88 89.154) (width 0.762) (layer F.Cu) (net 14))
 (segment (start 184.658 84.074) (end 184.658 87.376) (width 0.762) (layer F.Cu) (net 14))
 (segment (start 185.928 78.232) (end 192.278 78.232) (width 0.762) (layer F.Cu) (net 15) (status 1000000))
 (segment (start 192.278 78.232) (end 194.31 76.2) (width 0.762) (layer F.Cu) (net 15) (status 1000000))
 (segment (start 168.144 94.488) (end 167.894 94.488) (width 0.762) (layer F.Cu) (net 16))
 (segment (start 171.958 90.674) (end 168.144 94.488) (width 0.762) (layer F.Cu) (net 16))
 (segment (start 171.958 84.074) (end 171.958 90.674) (width 0.762) (layer F.Cu) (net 16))
 (segment (start 175.26 100.342) (end 175.26 101.854) (width 0.762) (layer F.Cu) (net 16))
 (segment (start 169.406 94.488) (end 175.26 100.342) (width 0.762) (layer F.Cu) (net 16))
 (segment (start 167.894 94.488) (end 169.406 94.488) (width 0.762) (layer F.Cu) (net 16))
 (segment (start 162.052 88.138) (end 162.052 95.758) (width 0.762) (layer F.Cu) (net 17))
 (segment (start 162.052 95.758) (end 167.894 95.758) (width 0.762) (layer F.Cu) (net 17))
 (segment (start 160.274 95.758) (end 154.432 101.6) (width 0.762) (layer F.Cu) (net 17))
 (segment (start 162.052 95.758) (end 160.274 95.758) (width 0.762) (layer F.Cu) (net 17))
 (segment (start 146.05 80.518) (end 146.05 77.47) (width 0.762) (layer F.Cu) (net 20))
 (segment (start 154.432 88.9) (end 146.05 80.518) (width 0.762) (layer F.Cu) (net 20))
 (segment (start 125.73 57.912) (end 125.73 84.074) (width 0.762) (layer F.Cu) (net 21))
 (segment (start 135.89 94.234) (end 135.89 101.6) (width 0.762) (layer F.Cu) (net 21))
 (segment (start 125.73 84.074) (end 135.89 94.234) (width 0.762) (layer F.Cu) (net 21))
 (segment (start 135.89 50.292) (end 130.81 45.212) (width 0.762) (layer F.Cu) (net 22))
 (segment (start 135.89 57.912) (end 135.89 50.292) (width 0.762) (layer F.Cu) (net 22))
 (segment (start 135.89 57.912) (end 135.89 64.008) (width 0.762) (layer F.Cu) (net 22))
 (segment (start 138.43 66.548) (end 138.43 69.85) (width 0.762) (layer F.Cu) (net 22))
 (segment (start 135.89 64.008) (end 138.43 66.548) (width 0.762) (layer F.Cu) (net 22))
 (segment (start 138.43 47.752) (end 135.89 45.212) (width 0.762) (layer F.Cu) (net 23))
 (segment (start 138.43 53.086) (end 138.43 47.752) (width 0.762) (layer F.Cu) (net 23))
 (segment (start 140.716 55.372) (end 138.43 53.086) (width 0.762) (layer F.Cu) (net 23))
 (segment (start 148.59 60.198) (end 143.764 55.372) (width 0.762) (layer F.Cu) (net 23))
 (segment (start 143.764 55.372) (end 140.716 55.372) (width 0.762) (layer F.Cu) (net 23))
 (segment (start 216.154 55.626) (end 216.154 60.706) (width 2.032) (layer F.Cu) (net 13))
 (segment (start 127.254 92.456) (end 123.698 88.9) (width 0.762) (layer F.Cu) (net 19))
 (segment (start 129.286 92.456) (end 127.254 92.456) (width 0.762) (layer F.Cu) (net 19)))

